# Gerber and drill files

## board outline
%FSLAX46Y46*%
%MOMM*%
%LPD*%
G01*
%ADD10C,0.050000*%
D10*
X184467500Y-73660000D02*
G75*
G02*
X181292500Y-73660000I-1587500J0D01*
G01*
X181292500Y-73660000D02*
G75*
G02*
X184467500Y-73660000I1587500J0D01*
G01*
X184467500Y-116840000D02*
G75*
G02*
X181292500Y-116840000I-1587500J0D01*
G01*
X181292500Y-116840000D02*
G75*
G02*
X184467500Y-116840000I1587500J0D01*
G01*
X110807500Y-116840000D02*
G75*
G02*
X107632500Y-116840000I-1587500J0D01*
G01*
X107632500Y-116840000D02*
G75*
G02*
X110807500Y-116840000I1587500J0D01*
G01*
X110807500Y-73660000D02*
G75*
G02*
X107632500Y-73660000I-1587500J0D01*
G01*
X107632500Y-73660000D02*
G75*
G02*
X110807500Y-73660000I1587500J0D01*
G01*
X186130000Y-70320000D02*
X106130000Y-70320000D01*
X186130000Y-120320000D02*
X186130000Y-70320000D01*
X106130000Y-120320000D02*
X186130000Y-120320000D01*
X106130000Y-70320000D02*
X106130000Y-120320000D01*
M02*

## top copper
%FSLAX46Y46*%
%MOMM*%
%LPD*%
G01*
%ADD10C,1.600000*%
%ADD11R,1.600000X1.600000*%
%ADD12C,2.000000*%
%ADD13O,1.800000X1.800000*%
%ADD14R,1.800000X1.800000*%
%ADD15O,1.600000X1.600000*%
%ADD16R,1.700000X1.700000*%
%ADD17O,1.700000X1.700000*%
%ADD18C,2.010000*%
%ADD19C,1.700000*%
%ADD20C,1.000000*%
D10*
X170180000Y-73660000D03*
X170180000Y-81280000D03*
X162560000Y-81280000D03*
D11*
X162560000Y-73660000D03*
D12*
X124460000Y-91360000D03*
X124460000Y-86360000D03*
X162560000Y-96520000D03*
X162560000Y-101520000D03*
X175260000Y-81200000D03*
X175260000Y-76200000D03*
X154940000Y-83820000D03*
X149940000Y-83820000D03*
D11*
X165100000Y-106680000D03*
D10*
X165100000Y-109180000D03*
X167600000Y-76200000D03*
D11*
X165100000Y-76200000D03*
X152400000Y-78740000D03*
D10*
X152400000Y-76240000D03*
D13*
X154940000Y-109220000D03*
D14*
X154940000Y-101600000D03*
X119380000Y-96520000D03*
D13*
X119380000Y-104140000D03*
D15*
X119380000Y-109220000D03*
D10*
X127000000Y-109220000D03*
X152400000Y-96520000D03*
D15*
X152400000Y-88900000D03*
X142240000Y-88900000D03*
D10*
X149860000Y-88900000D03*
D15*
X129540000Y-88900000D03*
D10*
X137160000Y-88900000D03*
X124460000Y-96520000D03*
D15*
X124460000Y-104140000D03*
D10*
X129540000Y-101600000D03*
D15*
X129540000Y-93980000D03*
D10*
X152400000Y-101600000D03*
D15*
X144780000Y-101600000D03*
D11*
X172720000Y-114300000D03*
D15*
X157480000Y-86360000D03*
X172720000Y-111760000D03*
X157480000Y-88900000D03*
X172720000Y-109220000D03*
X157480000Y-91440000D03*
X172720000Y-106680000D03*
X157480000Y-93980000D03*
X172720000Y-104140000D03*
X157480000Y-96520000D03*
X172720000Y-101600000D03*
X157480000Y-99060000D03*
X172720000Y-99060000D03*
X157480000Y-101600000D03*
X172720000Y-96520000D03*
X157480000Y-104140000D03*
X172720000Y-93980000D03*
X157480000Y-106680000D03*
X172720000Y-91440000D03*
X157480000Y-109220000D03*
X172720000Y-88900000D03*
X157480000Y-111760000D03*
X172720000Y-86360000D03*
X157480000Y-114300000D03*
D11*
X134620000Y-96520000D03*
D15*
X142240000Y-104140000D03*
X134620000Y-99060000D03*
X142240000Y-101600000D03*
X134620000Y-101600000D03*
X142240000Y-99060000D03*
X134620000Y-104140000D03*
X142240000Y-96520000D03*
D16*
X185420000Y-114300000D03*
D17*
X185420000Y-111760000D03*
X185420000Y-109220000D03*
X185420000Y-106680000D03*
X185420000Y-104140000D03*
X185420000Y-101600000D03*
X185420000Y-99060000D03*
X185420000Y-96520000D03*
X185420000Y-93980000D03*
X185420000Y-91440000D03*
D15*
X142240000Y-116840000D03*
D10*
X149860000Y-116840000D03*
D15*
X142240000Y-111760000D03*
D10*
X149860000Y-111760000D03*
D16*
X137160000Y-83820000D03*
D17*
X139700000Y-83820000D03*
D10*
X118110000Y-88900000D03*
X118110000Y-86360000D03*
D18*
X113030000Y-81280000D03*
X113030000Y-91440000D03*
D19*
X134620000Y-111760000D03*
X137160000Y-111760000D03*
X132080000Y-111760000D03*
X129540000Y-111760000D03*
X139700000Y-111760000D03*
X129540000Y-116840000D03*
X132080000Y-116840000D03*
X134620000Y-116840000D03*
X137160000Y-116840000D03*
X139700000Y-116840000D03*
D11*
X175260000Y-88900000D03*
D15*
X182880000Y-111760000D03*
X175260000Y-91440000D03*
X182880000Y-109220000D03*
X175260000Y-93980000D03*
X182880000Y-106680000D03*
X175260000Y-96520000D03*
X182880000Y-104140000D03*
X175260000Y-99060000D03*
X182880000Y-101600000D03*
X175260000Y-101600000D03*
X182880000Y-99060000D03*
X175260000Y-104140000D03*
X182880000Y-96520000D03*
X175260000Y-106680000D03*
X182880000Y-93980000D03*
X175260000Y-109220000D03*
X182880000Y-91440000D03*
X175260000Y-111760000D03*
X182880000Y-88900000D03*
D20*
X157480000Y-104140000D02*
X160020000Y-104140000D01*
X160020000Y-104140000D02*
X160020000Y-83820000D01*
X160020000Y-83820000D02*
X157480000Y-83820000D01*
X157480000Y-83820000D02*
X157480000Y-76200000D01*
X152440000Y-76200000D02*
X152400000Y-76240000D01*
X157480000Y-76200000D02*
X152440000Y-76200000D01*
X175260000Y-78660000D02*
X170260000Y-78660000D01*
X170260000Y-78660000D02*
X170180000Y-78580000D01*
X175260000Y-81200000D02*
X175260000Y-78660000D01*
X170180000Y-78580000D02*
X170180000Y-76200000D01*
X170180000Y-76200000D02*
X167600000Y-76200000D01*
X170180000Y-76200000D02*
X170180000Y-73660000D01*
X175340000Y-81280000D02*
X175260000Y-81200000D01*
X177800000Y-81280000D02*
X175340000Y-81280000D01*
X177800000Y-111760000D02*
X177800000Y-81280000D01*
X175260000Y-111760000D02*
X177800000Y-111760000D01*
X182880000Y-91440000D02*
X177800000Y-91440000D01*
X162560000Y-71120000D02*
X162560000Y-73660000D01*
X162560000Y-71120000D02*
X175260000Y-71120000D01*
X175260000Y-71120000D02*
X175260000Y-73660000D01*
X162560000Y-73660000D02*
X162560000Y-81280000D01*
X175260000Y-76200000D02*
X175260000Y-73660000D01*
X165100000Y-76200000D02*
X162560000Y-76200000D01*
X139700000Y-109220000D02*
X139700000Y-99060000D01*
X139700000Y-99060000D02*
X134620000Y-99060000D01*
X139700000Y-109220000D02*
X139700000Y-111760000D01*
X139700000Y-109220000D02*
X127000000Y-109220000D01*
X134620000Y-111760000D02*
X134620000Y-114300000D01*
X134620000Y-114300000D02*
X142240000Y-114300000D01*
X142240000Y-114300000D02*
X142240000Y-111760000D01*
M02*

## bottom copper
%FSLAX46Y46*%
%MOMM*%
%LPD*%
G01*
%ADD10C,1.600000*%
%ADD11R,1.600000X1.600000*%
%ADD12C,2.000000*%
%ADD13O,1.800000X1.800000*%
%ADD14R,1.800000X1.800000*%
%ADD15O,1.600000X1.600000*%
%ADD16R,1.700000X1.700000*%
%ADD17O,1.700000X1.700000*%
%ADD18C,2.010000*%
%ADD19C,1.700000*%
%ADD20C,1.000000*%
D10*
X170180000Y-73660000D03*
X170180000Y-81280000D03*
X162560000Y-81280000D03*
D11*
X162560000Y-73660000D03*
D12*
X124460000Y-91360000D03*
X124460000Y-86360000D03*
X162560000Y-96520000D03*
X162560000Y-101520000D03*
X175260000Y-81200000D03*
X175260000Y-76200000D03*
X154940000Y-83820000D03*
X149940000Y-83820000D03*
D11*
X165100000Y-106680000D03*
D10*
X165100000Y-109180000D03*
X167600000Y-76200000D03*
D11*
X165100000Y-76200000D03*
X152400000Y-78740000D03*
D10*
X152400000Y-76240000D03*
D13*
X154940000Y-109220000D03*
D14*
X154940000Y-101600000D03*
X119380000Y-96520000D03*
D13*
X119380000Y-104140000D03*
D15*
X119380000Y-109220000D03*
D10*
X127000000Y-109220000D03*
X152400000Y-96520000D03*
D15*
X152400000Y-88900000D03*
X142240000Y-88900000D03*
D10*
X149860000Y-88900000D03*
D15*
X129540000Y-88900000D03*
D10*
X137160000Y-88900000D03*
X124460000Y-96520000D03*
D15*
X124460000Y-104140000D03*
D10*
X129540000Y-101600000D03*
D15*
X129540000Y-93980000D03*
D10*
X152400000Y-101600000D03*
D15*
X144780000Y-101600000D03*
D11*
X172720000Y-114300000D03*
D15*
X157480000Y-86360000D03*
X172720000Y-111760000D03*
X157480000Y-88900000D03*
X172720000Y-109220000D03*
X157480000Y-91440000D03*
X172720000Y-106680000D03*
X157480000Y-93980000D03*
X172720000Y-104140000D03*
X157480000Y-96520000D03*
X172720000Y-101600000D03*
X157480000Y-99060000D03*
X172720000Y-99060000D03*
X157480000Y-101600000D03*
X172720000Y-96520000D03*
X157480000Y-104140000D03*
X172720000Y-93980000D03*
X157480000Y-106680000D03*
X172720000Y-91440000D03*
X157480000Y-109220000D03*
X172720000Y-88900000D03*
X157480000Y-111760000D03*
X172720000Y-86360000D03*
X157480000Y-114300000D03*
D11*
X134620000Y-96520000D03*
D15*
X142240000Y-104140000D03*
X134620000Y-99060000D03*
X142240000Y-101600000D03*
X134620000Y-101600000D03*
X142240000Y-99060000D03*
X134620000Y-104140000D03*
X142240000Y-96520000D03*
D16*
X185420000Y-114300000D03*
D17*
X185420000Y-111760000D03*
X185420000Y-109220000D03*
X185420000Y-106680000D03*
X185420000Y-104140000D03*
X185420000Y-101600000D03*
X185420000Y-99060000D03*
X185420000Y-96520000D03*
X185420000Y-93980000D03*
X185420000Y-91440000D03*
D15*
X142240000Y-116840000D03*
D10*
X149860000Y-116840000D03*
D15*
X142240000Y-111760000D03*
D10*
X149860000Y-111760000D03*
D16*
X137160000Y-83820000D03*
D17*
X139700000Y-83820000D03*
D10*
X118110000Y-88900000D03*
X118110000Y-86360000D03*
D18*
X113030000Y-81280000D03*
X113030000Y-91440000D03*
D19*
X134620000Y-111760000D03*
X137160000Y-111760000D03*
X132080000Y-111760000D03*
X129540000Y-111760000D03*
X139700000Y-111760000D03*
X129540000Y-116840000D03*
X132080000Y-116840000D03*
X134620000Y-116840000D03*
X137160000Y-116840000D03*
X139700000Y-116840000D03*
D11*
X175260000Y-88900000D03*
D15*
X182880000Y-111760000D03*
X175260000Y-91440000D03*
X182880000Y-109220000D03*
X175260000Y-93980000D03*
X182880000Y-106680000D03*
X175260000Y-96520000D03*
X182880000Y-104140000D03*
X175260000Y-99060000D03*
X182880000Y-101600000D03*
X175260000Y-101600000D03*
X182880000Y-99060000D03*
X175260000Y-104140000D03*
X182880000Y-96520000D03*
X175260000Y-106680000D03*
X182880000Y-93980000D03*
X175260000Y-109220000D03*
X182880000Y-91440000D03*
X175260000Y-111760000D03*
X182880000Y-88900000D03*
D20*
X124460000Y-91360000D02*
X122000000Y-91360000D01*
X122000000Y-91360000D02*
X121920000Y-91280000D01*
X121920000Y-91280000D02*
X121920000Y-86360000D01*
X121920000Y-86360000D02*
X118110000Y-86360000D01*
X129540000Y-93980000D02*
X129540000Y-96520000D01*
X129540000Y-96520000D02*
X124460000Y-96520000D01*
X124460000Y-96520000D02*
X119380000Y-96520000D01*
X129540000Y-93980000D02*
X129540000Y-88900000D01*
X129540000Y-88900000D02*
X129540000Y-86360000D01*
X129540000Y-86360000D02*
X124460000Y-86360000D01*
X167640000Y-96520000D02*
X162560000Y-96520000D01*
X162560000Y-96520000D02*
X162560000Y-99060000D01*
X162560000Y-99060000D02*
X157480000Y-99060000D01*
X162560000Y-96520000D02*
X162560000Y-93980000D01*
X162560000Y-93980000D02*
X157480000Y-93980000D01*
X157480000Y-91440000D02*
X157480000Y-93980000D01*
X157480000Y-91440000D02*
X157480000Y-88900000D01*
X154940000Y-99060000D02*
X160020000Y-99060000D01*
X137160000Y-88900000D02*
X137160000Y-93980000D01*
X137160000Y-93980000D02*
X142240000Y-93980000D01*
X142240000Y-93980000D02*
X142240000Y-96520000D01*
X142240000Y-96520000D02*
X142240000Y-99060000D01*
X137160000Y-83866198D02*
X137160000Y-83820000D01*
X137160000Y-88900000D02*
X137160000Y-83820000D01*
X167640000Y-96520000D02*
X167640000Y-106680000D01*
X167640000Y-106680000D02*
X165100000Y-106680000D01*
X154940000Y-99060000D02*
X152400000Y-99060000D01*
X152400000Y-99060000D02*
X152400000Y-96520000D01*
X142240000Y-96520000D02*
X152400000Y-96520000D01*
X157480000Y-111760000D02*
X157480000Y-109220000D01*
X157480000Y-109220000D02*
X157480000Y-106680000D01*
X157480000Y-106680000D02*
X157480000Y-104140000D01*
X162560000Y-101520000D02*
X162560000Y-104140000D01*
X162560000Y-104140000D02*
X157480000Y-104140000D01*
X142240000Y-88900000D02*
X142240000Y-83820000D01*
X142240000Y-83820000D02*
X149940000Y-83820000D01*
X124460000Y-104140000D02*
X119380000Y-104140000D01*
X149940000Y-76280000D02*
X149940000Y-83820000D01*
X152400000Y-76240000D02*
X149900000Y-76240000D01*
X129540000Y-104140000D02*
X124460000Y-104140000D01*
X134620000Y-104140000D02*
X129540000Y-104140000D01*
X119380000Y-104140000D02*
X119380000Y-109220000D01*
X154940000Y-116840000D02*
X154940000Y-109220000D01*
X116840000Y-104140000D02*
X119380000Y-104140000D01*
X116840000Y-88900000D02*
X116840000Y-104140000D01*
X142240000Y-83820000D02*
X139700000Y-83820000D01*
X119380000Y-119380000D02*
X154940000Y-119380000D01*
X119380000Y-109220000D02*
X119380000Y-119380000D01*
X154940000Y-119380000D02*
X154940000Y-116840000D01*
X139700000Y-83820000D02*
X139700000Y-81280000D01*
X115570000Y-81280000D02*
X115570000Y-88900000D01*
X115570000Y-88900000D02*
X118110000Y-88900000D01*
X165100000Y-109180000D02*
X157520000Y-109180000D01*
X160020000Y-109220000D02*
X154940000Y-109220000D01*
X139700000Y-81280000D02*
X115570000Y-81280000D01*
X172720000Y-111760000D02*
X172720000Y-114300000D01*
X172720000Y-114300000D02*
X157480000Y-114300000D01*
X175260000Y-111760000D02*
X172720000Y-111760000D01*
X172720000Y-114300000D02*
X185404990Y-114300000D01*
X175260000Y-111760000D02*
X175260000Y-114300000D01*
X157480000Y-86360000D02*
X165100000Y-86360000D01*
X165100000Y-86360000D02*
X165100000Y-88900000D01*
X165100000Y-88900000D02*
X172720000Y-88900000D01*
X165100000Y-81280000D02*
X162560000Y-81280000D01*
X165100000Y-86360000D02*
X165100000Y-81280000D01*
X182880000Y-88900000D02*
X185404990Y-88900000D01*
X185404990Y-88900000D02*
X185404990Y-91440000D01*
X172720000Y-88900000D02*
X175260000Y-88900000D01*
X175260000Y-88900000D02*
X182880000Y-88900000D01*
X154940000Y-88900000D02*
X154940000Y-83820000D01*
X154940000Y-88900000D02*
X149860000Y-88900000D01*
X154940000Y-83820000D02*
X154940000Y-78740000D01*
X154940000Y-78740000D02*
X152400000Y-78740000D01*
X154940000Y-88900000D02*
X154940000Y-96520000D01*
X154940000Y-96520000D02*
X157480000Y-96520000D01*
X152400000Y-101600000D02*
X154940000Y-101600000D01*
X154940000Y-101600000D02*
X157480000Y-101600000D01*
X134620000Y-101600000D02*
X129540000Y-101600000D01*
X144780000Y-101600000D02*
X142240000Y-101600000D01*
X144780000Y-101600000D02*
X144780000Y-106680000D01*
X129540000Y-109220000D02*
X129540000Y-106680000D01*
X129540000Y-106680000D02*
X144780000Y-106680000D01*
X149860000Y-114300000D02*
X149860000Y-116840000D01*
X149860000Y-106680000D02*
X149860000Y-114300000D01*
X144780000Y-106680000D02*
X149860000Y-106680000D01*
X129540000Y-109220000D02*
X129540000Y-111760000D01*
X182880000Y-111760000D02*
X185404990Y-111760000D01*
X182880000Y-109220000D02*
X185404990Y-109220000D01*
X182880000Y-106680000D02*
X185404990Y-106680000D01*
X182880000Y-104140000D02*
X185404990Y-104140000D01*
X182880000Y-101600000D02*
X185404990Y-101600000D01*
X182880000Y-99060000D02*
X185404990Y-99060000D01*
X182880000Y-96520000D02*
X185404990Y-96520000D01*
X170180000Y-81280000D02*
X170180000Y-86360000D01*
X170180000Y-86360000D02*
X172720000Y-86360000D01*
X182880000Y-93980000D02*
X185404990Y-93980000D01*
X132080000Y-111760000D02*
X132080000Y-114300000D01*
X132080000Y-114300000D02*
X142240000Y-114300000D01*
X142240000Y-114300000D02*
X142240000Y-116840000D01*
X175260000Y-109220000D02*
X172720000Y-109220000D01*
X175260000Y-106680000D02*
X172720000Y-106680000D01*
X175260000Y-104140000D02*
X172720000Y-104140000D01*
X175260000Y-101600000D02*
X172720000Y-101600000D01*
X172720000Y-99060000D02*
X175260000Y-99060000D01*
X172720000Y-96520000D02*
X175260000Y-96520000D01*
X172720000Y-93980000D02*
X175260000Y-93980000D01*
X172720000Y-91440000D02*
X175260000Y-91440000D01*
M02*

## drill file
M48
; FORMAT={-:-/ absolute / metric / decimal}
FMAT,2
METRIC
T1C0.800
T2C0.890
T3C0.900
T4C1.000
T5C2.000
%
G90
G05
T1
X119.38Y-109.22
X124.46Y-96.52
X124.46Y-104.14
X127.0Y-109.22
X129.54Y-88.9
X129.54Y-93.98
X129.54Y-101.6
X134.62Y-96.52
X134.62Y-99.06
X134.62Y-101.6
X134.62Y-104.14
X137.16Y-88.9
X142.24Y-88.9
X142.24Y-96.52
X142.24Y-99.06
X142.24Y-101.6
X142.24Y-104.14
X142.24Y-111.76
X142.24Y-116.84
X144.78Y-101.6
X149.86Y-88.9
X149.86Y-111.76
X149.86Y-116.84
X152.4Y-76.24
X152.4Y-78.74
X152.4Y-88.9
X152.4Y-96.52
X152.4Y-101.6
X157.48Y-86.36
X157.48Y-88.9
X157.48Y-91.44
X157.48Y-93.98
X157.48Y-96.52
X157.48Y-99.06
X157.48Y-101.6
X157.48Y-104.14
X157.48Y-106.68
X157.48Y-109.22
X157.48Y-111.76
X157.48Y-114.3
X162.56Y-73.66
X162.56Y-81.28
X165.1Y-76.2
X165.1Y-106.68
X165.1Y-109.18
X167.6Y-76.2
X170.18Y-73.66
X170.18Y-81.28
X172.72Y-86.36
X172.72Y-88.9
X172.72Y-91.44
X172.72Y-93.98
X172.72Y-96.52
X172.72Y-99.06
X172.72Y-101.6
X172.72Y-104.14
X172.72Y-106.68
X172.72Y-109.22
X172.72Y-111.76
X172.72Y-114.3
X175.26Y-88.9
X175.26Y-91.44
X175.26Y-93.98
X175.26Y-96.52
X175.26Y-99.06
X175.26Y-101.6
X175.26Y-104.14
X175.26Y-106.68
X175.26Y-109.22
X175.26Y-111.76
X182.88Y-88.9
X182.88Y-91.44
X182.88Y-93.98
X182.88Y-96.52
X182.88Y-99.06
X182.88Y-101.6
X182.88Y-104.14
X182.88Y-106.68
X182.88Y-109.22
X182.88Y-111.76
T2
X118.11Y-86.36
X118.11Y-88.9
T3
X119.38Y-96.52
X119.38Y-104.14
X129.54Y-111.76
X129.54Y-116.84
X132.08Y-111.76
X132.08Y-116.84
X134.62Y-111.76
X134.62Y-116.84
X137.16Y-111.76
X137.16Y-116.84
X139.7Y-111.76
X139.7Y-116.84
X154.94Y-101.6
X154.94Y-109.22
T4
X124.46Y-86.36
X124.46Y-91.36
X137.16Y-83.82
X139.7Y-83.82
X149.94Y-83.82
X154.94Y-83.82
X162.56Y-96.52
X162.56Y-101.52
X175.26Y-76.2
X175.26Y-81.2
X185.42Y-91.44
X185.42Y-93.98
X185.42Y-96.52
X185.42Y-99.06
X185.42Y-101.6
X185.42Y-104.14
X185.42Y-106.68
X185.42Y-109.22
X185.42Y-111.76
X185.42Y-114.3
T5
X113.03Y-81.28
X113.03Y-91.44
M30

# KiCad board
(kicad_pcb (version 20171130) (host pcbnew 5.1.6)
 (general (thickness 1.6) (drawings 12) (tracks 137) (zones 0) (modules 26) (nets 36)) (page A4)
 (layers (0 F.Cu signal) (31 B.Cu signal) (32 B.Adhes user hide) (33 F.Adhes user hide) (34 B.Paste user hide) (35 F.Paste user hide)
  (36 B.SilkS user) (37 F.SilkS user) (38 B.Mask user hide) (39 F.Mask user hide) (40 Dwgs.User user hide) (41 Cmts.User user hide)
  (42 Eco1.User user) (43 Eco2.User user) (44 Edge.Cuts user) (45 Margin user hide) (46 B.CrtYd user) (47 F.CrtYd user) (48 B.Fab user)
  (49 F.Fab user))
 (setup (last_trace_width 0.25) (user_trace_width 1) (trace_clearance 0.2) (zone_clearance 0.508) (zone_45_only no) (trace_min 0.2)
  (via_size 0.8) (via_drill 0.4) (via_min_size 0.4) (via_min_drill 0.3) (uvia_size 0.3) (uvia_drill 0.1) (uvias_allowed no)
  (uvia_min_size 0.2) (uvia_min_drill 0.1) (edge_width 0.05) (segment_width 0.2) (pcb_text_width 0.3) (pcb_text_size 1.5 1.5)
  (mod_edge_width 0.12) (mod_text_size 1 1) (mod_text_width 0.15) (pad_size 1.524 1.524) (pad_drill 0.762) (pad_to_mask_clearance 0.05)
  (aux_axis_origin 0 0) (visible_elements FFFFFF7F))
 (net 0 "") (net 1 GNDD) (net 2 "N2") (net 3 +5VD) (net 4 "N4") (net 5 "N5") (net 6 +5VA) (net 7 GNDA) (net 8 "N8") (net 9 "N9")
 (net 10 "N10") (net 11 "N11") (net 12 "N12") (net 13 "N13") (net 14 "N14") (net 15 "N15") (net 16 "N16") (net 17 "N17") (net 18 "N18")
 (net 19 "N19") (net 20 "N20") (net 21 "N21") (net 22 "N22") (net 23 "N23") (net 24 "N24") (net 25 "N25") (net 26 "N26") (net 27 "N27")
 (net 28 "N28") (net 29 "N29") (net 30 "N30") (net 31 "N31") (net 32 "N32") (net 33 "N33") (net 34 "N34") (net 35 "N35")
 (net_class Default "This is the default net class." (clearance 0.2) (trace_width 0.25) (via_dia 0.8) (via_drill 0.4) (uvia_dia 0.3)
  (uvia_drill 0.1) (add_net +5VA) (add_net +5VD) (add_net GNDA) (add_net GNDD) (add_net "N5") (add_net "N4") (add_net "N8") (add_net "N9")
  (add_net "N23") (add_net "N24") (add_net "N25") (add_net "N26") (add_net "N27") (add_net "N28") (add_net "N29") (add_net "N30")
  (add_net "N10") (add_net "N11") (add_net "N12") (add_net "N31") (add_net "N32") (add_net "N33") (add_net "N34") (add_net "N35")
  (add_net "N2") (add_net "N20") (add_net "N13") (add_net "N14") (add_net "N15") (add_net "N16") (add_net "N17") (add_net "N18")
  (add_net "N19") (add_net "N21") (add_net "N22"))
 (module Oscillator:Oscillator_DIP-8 (layer B.Cu) (at 162.56 73.66)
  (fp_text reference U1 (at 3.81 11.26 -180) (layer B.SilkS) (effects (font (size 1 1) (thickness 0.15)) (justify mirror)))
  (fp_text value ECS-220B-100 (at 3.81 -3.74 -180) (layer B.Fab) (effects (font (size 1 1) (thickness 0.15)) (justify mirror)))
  (pad 4 thru_hole circle (at 7.62 0) (size 1.6 1.6) (drill 0.8) (layers *.Cu *.Mask) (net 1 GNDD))
  (pad 5 thru_hole circle (at 7.62 7.62) (size 1.6 1.6) (drill 0.8) (layers *.Cu *.Mask) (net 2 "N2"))
  (pad 8 thru_hole circle (at 0 7.62) (size 1.6 1.6) (drill 0.8) (layers *.Cu *.Mask) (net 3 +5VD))
  (pad 1 thru_hole rect (at 0 0) (size 1.6 1.6) (drill 0.8) (layers *.Cu *.Mask) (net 3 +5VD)))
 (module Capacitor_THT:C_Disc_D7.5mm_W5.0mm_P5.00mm (layer F.Cu) (at 124.46 86.36 270)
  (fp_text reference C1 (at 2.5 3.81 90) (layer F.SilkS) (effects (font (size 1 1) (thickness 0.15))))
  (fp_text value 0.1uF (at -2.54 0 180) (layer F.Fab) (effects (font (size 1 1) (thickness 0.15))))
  (pad 2 thru_hole circle (at 5 0 270) (size 2 2) (drill 1) (layers *.Cu *.Mask) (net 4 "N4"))
  (pad 1 thru_hole circle (at 0 0 270) (size 2 2) (drill 1) (layers *.Cu *.Mask) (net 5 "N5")))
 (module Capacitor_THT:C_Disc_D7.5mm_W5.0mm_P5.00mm (layer B.Cu) (at 162.56 96.52 270)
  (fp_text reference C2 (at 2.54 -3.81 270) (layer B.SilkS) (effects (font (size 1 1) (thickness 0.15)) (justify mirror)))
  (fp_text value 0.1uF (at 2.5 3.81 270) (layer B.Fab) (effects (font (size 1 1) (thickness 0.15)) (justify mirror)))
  (pad 1 thru_hole circle (at 0 0 270) (size 2 2) (drill 1) (layers *.Cu *.Mask) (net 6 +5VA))
  (pad 2 thru_hole circle (at 5 0 270) (size 2 2) (drill 1) (layers *.Cu *.Mask) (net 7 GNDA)))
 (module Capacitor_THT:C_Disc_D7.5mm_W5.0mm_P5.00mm (layer F.Cu) (at 175.26 76.2 270)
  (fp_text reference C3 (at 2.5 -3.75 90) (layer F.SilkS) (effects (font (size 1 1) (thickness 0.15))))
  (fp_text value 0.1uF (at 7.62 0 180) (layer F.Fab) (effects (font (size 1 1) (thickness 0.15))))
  (pad 2 thru_hole circle (at 5 0 270) (size 2 2) (drill 1) (layers *.Cu *.Mask) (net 1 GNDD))
  (pad 1 thru_hole circle (at 0 0 270) (size 2 2) (drill 1) (layers *.Cu *.Mask) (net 3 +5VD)))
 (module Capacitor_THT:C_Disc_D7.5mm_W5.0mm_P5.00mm (layer F.Cu) (at 154.94 83.82 180)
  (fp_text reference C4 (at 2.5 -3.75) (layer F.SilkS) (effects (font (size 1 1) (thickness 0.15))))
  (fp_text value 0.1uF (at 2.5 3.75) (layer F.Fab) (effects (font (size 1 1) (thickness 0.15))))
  (pad 1 thru_hole circle (at 0 0 180) (size 2 2) (drill 1) (layers *.Cu *.Mask) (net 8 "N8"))
  (pad 2 thru_hole circle (at 5 0 180) (size 2 2) (drill 1) (layers *.Cu *.Mask) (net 7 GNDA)))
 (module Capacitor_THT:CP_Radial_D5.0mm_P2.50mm (layer B.Cu) (at 165.1 106.68 270)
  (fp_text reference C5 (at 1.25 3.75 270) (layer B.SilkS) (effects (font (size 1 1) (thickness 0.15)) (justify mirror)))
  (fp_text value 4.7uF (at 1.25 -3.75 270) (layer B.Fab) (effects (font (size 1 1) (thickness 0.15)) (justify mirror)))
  (pad 1 thru_hole rect (at 0 0 270) (size 1.6 1.6) (drill 0.8) (layers *.Cu *.Mask) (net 6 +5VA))
  (pad 2 thru_hole circle (at 2.5 0 270) (size 1.6 1.6) (drill 0.8) (layers *.Cu *.Mask) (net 7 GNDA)))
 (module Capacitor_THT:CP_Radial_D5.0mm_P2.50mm (layer F.Cu) (at 165.1 76.2)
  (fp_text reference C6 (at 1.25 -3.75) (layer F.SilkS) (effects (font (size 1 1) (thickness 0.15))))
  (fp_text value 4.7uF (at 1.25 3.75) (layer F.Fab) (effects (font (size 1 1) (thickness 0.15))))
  (pad 2 thru_hole circle (at 2.5 0) (size 1.6 1.6) (drill 0.8) (layers *.Cu *.Mask) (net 1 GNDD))
  (pad 1 thru_hole rect (at 0 0) (size 1.6 1.6) (drill 0.8) (layers *.Cu *.Mask) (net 3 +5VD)))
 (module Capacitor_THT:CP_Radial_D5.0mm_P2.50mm (layer F.Cu) (at 152.4 78.74 90)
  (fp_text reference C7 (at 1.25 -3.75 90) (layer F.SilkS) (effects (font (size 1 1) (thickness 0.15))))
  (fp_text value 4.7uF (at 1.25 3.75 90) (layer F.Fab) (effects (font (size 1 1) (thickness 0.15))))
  (pad 1 thru_hole rect (at 0 0 90) (size 1.6 1.6) (drill 0.8) (layers *.Cu *.Mask) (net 8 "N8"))
  (pad 2 thru_hole circle (at 2.5 0 90) (size 1.6 1.6) (drill 0.8) (layers *.Cu *.Mask) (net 7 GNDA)))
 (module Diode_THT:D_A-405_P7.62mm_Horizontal (layer F.Cu) (at 154.94 101.6 270)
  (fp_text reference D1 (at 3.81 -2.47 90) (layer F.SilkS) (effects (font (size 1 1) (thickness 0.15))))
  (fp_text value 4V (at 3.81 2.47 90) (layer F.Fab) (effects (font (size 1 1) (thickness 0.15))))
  (pad 2 thru_hole oval (at 7.62 0 270) (size 1.8 1.8) (drill 0.9) (layers *.Cu *.Mask) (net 7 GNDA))
  (pad 1 thru_hole rect (at 0 0 270) (size 1.8 1.8) (drill 0.9) (layers *.Cu *.Mask) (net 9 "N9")))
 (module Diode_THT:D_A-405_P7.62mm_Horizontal (layer F.Cu) (at 119.38 96.52 270)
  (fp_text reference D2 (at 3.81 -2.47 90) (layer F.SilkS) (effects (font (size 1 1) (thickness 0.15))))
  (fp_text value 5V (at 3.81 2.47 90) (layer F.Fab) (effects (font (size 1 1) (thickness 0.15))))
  (pad 1 thru_hole rect (at 0 0 270) (size 1.8 1.8) (drill 0.9) (layers *.Cu *.Mask) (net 5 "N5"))
  (pad 2 thru_hole oval (at 7.62 0 270) (size 1.8 1.8) (drill 0.9) (layers *.Cu *.Mask) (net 7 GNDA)))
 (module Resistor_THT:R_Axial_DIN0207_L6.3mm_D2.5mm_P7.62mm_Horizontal (layer F.Cu) (at 127 109.22 180)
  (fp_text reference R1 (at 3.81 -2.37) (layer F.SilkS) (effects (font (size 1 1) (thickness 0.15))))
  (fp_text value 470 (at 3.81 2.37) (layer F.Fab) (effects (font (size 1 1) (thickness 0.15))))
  (pad 2 thru_hole oval (at 7.62 0 180) (size 1.6 1.6) (drill 0.8) (layers *.Cu *.Mask) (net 7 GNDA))
  (pad 1 thru_hole circle (at 0 0 180) (size 1.6 1.6) (drill 0.8) (layers *.Cu *.Mask) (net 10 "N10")))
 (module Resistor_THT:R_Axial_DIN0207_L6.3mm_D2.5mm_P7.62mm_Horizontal (layer F.Cu) (at 152.4 96.52 90)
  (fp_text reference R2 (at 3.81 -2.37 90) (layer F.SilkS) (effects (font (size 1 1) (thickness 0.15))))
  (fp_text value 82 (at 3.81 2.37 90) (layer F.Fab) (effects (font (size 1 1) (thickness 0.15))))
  (pad 1 thru_hole circle (at 0 0 90) (size 1.6 1.6) (drill 0.8) (layers *.Cu *.Mask) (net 6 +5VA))
  (pad 2 thru_hole oval (at 7.62 0 90) (size 1.6 1.6) (drill 0.8) (layers *.Cu *.Mask) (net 8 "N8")))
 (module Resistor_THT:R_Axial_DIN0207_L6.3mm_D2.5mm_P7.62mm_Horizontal (layer F.Cu) (at 149.86 88.9 180)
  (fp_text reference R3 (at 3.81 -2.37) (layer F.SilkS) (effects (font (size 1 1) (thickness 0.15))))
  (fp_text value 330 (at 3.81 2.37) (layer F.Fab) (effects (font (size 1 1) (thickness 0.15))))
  (pad 2 thru_hole oval (at 7.62 0 180) (size 1.6 1.6) (drill 0.8) (layers *.Cu *.Mask) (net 7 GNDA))
  (pad 1 thru_hole circle (at 0 0 180) (size 1.6 1.6) (drill 0.8) (layers *.Cu *.Mask) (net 8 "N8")))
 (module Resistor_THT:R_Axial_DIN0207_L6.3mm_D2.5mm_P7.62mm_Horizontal (layer F.Cu) (at 137.16 88.9 180)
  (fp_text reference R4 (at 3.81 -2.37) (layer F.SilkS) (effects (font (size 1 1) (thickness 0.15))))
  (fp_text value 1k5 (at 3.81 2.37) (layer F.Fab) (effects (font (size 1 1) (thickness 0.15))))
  (pad 2 thru_hole oval (at 7.62 0 180) (size 1.6 1.6) (drill 0.8) (layers *.Cu *.Mask) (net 5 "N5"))
  (pad 1 thru_hole circle (at 0 0 180) (size 1.6 1.6) (drill 0.8) (layers *.Cu *.Mask) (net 6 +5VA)))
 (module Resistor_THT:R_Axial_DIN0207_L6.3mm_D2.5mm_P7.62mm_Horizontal (layer F.Cu) (at 124.46 96.52 270)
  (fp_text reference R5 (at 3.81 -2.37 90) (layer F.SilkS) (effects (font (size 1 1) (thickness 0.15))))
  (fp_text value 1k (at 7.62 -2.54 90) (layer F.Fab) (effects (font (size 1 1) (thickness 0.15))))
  (pad 1 thru_hole circle (at 0 0 270) (size 1.6 1.6) (drill 0.8) (layers *.Cu *.Mask) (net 5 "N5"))
  (pad 2 thru_hole oval (at 7.62 0 270) (size 1.6 1.6) (drill 0.8) (layers *.Cu *.Mask) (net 7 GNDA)))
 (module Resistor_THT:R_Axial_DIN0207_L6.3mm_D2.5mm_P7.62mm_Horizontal (layer F.Cu) (at 129.54 101.6 90)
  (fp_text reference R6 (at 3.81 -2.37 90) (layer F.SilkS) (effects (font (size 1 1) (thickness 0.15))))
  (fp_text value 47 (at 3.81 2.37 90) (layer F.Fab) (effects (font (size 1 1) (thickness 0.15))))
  (pad 1 thru_hole circle (at 0 0 90) (size 1.6 1.6) (drill 0.8) (layers *.Cu *.Mask) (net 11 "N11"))
  (pad 2 thru_hole oval (at 7.62 0 90) (size 1.6 1.6) (drill 0.8) (layers *.Cu *.Mask) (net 5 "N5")))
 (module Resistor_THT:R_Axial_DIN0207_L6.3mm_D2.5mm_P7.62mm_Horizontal (layer F.Cu) (at 152.4 101.6 180)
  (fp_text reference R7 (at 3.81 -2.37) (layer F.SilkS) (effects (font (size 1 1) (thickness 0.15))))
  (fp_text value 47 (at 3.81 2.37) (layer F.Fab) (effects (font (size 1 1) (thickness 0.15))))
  (pad 1 thru_hole circle (at 0 0 180) (size 1.6 1.6) (drill 0.8) (layers *.Cu *.Mask) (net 9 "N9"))
  (pad 2 thru_hole oval (at 7.62 0 180) (size 1.6 1.6) (drill 0.8) (layers *.Cu *.Mask) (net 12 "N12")))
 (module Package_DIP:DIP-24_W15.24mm (layer F.Cu) (at 172.72 114.3 180)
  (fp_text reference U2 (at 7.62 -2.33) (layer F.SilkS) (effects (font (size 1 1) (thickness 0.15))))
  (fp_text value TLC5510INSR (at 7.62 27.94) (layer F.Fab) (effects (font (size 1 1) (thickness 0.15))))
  (pad 1 thru_hole rect (at 0 0 180) (size 1.6 1.6) (drill 0.8) (layers *.Cu *.Mask) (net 1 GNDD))
  (pad 13 thru_hole oval (at 15.24 27.94 180) (size 1.6 1.6) (drill 0.8) (layers *.Cu *.Mask) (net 3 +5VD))
  (pad 2 thru_hole oval (at 0 2.54 180) (size 1.6 1.6) (drill 0.8) (layers *.Cu *.Mask) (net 1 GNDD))
  (pad 14 thru_hole oval (at 15.24 25.4 180) (size 1.6 1.6) (drill 0.8) (layers *.Cu *.Mask) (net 6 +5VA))
  (pad 3 thru_hole oval (at 0 5.08 180) (size 1.6 1.6) (drill 0.8) (layers *.Cu *.Mask) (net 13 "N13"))
  (pad 15 thru_hole oval (at 15.24 22.86 180) (size 1.6 1.6) (drill 0.8) (layers *.Cu *.Mask) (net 6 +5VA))
  (pad 4 thru_hole oval (at 0 7.62 180) (size 1.6 1.6) (drill 0.8) (layers *.Cu *.Mask) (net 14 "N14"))
  (pad 16 thru_hole oval (at 15.24 20.32 180) (size 1.6 1.6) (drill 0.8) (layers *.Cu *.Mask) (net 6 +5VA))
  (pad 5 thru_hole oval (at 0 10.16 180) (size 1.6 1.6) (drill 0.8) (layers *.Cu *.Mask) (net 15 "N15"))
  (pad 17 thru_hole oval (at 15.24 17.78 180) (size 1.6 1.6) (drill 0.8) (layers *.Cu *.Mask) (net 8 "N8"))
  (pad 6 thru_hole oval (at 0 12.7 180) (size 1.6 1.6) (drill 0.8) (layers *.Cu *.Mask) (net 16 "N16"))
  (pad 18 thru_hole oval (at 15.24 15.24 180) (size 1.6 1.6) (drill 0.8) (layers *.Cu *.Mask) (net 6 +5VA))
  (pad 7 thru_hole oval (at 0 15.24 180) (size 1.6 1.6) (drill 0.8) (layers *.Cu *.Mask) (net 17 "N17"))
  (pad 19 thru_hole oval (at 15.24 12.7 180) (size 1.6 1.6) (drill 0.8) (layers *.Cu *.Mask) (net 9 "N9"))
  (pad 8 thru_hole oval (at 0 17.78 180) (size 1.6 1.6) (drill 0.8) (layers *.Cu *.Mask) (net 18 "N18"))
  (pad 20 thru_hole oval (at 15.24 10.16 180) (size 1.6 1.6) (drill 0.8) (layers *.Cu *.Mask) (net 7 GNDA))
  (pad 9 thru_hole oval (at 0 20.32 180) (size 1.6 1.6) (drill 0.8) (layers *.Cu *.Mask) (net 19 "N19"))
  (pad 21 thru_hole oval (at 15.24 7.62 180) (size 1.6 1.6) (drill 0.8) (layers *.Cu *.Mask) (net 7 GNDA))
  (pad 10 thru_hole oval (at 0 22.86 180) (size 1.6 1.6) (drill 0.8) (layers *.Cu *.Mask) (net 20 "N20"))
  (pad 22 thru_hole oval (at 15.24 5.08 180) (size 1.6 1.6) (drill 0.8) (layers *.Cu *.Mask) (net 7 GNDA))
  (pad 11 thru_hole oval (at 0 25.4 180) (size 1.6 1.6) (drill 0.8) (layers *.Cu *.Mask) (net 3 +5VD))
  (pad 23 thru_hole oval (at 15.24 2.54 180) (size 1.6 1.6) (drill 0.8) (layers *.Cu *.Mask) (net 7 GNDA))
  (pad 12 thru_hole oval (at 0 27.94 180) (size 1.6 1.6) (drill 0.8) (layers *.Cu *.Mask) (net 2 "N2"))
  (pad 24 thru_hole oval (at 15.24 0 180) (size 1.6 1.6) (drill 0.8) (layers *.Cu *.Mask) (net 1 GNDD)))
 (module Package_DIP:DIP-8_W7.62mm (layer F.Cu) (at 134.62 96.52)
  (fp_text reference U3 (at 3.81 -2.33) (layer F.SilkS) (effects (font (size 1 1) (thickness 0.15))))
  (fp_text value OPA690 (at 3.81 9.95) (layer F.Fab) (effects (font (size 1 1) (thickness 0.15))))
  (pad 1 thru_hole rect (at 0 0) (size 1.6 1.6) (drill 0.8) (layers *.Cu *.Mask) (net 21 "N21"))
  (pad 5 thru_hole oval (at 7.62 7.62) (size 1.6 1.6) (drill 0.8) (layers *.Cu *.Mask) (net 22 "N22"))
  (pad 2 thru_hole oval (at 0 2.54) (size 1.6 1.6) (drill 0.8) (layers *.Cu *.Mask) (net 10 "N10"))
  (pad 6 thru_hole oval (at 7.62 5.08) (size 1.6 1.6) (drill 0.8) (layers *.Cu *.Mask) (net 12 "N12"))
  (pad 3 thru_hole oval (at 0 5.08) (size 1.6 1.6) (drill 0.8) (layers *.Cu *.Mask) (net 11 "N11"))
  (pad 7 thru_hole oval (at 7.62 2.54) (size 1.6 1.6) (drill 0.8) (layers *.Cu *.Mask) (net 6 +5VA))
  (pad 4 thru_hole oval (at 0 7.62) (size 1.6 1.6) (drill 0.8) (layers *.Cu *.Mask) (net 7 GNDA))
  (pad 8 thru_hole oval (at 7.62 0) (size 1.6 1.6) (drill 0.8) (layers *.Cu *.Mask) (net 6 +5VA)))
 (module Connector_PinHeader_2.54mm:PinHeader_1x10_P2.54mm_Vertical (layer F.Cu) (at 185.42 114.3 180)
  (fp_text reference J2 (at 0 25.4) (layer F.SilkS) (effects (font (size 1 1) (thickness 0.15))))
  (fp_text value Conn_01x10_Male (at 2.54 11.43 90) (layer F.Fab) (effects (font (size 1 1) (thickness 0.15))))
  (pad 1 thru_hole rect (at 0 0 180) (size 1.7 1.7) (drill 1) (layers *.Cu *.Mask) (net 1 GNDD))
  (pad 2 thru_hole oval (at 0 2.54 180) (size 1.7 1.7) (drill 1) (layers *.Cu *.Mask) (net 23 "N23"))
  (pad 3 thru_hole oval (at 0 5.08 180) (size 1.7 1.7) (drill 1) (layers *.Cu *.Mask) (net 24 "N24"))
  (pad 4 thru_hole oval (at 0 7.62 180) (size 1.7 1.7) (drill 1) (layers *.Cu *.Mask) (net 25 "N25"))
  (pad 5 thru_hole oval (at 0 10.16 180) (size 1.7 1.7) (drill 1) (layers *.Cu *.Mask) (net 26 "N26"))
  (pad 6 thru_hole oval (at 0 12.7 180) (size 1.7 1.7) (drill 1) (layers *.Cu *.Mask) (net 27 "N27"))
  (pad 7 thru_hole oval (at 0 15.24 180) (size 1.7 1.7) (drill 1) (layers *.Cu *.Mask) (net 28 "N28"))
  (pad 8 thru_hole oval (at 0 17.78 180) (size 1.7 1.7) (drill 1) (layers *.Cu *.Mask) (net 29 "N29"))
  (pad 9 thru_hole oval (at 0 20.32 180) (size 1.7 1.7) (drill 1) (layers *.Cu *.Mask) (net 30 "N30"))
  (pad 10 thru_hole oval (at 0 22.86 180) (size 1.7 1.7) (drill 1) (layers *.Cu *.Mask) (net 3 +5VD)))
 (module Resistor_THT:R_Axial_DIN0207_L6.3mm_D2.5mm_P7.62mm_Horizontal (layer F.Cu) (at 149.86 116.84 180)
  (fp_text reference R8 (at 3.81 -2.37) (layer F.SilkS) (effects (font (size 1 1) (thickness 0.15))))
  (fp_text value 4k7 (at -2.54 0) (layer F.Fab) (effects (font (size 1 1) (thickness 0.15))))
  (pad 2 thru_hole oval (at 7.62 0 180) (size 1.6 1.6) (drill 0.8) (layers *.Cu *.Mask) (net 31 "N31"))
  (pad 1 thru_hole circle (at 0 0 180) (size 1.6 1.6) (drill 0.8) (layers *.Cu *.Mask) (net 12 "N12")))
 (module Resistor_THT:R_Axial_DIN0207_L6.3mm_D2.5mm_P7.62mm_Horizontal (layer F.Cu) (at 149.86 111.76 180)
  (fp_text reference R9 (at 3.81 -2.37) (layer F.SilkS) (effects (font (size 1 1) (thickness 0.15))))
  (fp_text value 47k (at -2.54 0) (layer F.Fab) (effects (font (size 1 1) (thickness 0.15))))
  (pad 2 thru_hole oval (at 7.62 0 180) (size 1.6 1.6) (drill 0.8) (layers *.Cu *.Mask) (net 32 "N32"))
  (pad 1 thru_hole circle (at 0 0 180) (size 1.6 1.6) (drill 0.8) (layers *.Cu *.Mask) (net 12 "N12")))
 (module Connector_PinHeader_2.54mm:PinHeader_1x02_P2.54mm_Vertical (layer F.Cu) (at 137.16 83.82 90)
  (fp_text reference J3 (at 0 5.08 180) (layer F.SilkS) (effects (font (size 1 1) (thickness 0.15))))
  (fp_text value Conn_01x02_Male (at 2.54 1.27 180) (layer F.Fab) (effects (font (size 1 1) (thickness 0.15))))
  (pad 1 thru_hole rect (at 0 0 90) (size 1.7 1.7) (drill 1) (layers *.Cu *.Mask) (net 6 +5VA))
  (pad 2 thru_hole oval (at 0 2.54 90) (size 1.7 1.7) (drill 1) (layers *.Cu *.Mask) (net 7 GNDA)))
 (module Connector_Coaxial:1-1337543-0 (layer F.Cu) (at 118.11 86.36 90)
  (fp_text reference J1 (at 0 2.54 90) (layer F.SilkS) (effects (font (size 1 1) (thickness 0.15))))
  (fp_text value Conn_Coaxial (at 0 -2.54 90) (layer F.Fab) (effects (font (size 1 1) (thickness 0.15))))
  (pad 2 thru_hole circle (at -2.54 0 90) (size 1.6 1.6) (drill 0.89) (layers *.Cu *.Mask) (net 7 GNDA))
  (pad 1 thru_hole circle (at 0 0 90) (size 1.6 1.6) (drill 0.89) (layers *.Cu *.Mask) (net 4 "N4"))
  (pad 4 thru_hole circle (at 5.08 -5.08 90) (size 2.01 2.01) (drill 2) (layers *.Cu *.Mask))
  (pad 3 thru_hole circle (at -5.08 -5.08 90) (size 2.01 2.01) (drill 2) (layers *.Cu *.Mask)))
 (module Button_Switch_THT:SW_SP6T (layer F.Cu) (at 134.62 111.76)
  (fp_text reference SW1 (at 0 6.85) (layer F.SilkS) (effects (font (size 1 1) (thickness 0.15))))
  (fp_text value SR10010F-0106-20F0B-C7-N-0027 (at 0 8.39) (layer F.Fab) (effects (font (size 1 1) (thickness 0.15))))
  (pad 3 thru_hole circle (at 0 0) (size 1.7 1.7) (drill 0.9) (layers *.Cu *.Mask) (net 32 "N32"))
  (pad 4 thru_hole circle (at 2.54 0) (size 1.7 1.7) (drill 0.9) (layers *.Cu *.Mask) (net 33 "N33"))
  (pad 2 thru_hole circle (at -2.54 0) (size 1.7 1.7) (drill 0.9) (layers *.Cu *.Mask) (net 31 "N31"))
  (pad 1 thru_hole circle (at -5.08 0) (size 1.7 1.7) (drill 0.9) (layers *.Cu *.Mask) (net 12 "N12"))
  (pad 5 thru_hole circle (at 5.08 0) (size 1.7 1.7) (drill 0.9) (layers *.Cu *.Mask) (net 10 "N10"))
  (pad 6 thru_hole circle (at -5.08 5.08) (size 1.7 1.7) (drill 0.9) (layers *.Cu *.Mask) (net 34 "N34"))
  (pad 7 thru_hole circle (at -2.54 5.08) (size 1.7 1.7) (drill 0.9) (layers *.Cu *.Mask) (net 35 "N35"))
  (pad 8 thru_hole circle (at 0 5.08) (size 1.7 1.7) (drill 0.9) (layers *.Cu *.Mask))
  (pad 9 thru_hole circle (at 2.54 5.08) (size 1.7 1.7) (drill 0.9) (layers *.Cu *.Mask))
  (pad 10 thru_hole circle (at 5.08 5.08) (size 1.7 1.7) (drill 0.9) (layers *.Cu *.Mask)))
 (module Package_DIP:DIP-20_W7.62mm (layer F.Cu) (at 175.26 88.9)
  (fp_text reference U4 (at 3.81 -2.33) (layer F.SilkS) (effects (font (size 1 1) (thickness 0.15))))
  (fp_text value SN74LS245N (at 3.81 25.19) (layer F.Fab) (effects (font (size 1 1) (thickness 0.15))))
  (pad 1 thru_hole rect (at 0 0) (size 1.6 1.6) (drill 0.8) (layers *.Cu *.Mask) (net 3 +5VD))
  (pad 11 thru_hole oval (at 7.62 22.86) (size 1.6 1.6) (drill 0.8) (layers *.Cu *.Mask) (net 23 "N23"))
  (pad 2 thru_hole oval (at 0 2.54) (size 1.6 1.6) (drill 0.8) (layers *.Cu *.Mask) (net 20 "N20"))
  (pad 12 thru_hole oval (at 7.62 20.32) (size 1.6 1.6) (drill 0.8) (layers *.Cu *.Mask) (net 24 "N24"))
  (pad 3 thru_hole oval (at 0 5.08) (size 1.6 1.6) (drill 0.8) (layers *.Cu *.Mask) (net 19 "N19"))
  (pad 13 thru_hole oval (at 7.62 17.78) (size 1.6 1.6) (drill 0.8) (layers *.Cu *.Mask) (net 25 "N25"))
  (pad 4 thru_hole oval (at 0 7.62) (size 1.6 1.6) (drill 0.8) (layers *.Cu *.Mask) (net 18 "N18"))
  (pad 14 thru_hole oval (at 7.62 15.24) (size 1.6 1.6) (drill 0.8) (layers *.Cu *.Mask) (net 26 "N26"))
  (pad 5 thru_hole oval (at 0 10.16) (size 1.6 1.6) (drill 0.8) (layers *.Cu *.Mask) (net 17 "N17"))
  (pad 15 thru_hole oval (at 7.62 12.7) (size 1.6 1.6) (drill 0.8) (layers *.Cu *.Mask) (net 27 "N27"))
  (pad 6 thru_hole oval (at 0 12.7) (size 1.6 1.6) (drill 0.8) (layers *.Cu *.Mask) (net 16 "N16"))
  (pad 16 thru_hole oval (at 7.62 10.16) (size 1.6 1.6) (drill 0.8) (layers *.Cu *.Mask) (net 28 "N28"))
  (pad 7 thru_hole oval (at 0 15.24) (size 1.6 1.6) (drill 0.8) (layers *.Cu *.Mask) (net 15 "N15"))
  (pad 17 thru_hole oval (at 7.62 7.62) (size 1.6 1.6) (drill 0.8) (layers *.Cu *.Mask) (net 29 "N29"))
  (pad 8 thru_hole oval (at 0 17.78) (size 1.6 1.6) (drill 0.8) (layers *.Cu *.Mask) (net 14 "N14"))
  (pad 18 thru_hole oval (at 7.62 5.08) (size 1.6 1.6) (drill 0.8) (layers *.Cu *.Mask) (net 30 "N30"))
  (pad 9 thru_hole oval (at 0 20.32) (size 1.6 1.6) (drill 0.8) (layers *.Cu *.Mask) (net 13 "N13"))
  (pad 19 thru_hole oval (at 7.62 2.54) (size 1.6 1.6) (drill 0.8) (layers *.Cu *.Mask) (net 1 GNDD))
  (pad 10 thru_hole oval (at 0 22.86) (size 1.6 1.6) (drill 0.8) (layers *.Cu *.Mask) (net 1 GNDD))
  (pad 20 thru_hole oval (at 7.62 0) (size 1.6 1.6) (drill 0.8) (layers *.Cu *.Mask) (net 3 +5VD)))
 (gr_circle (center 182.88 73.66) (end 184.4675 73.66) (layer Edge.Cuts) (width 0.05))
 (gr_circle (center 182.88 116.84) (end 184.4675 116.84) (layer Edge.Cuts) (width 0.05))
 (gr_circle (center 109.22 116.84) (end 110.8075 116.84) (layer Edge.Cuts) (width 0.05))
 (gr_circle (center 109.22 73.66) (end 110.8075 73.66) (layer Edge.Cuts) (width 0.05))
 (gr_line (start 186.13 70.32) (end 106.13 70.32) (layer Edge.Cuts) (width 0.05))
 (gr_line (start 186.13 120.32) (end 186.13 70.32) (layer Edge.Cuts) (width 0.05))
 (gr_line (start 106.13 120.32) (end 186.13 120.32) (layer Edge.Cuts) (width 0.05))
 (gr_line (start 106.13 70.32) (end 106.13 120.32) (layer Edge.Cuts) (width 0.05))
 (segment (start 124.46 91.36) (end 122 91.36) (width 1) (layer B.Cu) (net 4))
 (segment (start 122 91.36) (end 121.92 91.28) (width 1) (layer B.Cu) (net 4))
 (segment (start 121.92 91.28) (end 121.92 86.36) (width 1) (layer B.Cu) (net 4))
 (segment (start 121.92 86.36) (end 118.11 86.36) (width 1) (layer B.Cu) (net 4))
 (segment (start 129.54 93.98) (end 129.54 96.52) (width 1) (layer B.Cu) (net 5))
 (segment (start 129.54 96.52) (end 124.46 96.52) (width 1) (layer B.Cu) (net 5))
 (segment (start 124.46 96.52) (end 119.38 96.52) (width 1) (layer B.Cu) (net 5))
 (segment (start 129.54 93.98) (end 129.54 88.9) (width 1) (layer B.Cu) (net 5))
 (segment (start 129.54 88.9) (end 129.54 86.36) (width 1) (layer B.Cu) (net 5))
 (segment (start 129.54 86.36) (end 124.46 86.36) (width 1) (layer B.Cu) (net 5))
 (segment (start 167.64 96.52) (end 162.56 96.52) (width 1) (layer B.Cu) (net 6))
 (segment (start 162.56 96.52) (end 162.56 99.06) (width 1) (layer B.Cu) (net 6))
 (segment (start 162.56 99.06) (end 157.48 99.06) (width 1) (layer B.Cu) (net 6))
 (segment (start 162.56 96.52) (end 162.56 93.98) (width 1) (layer B.Cu) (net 6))
 (segment (start 162.56 93.98) (end 157.48 93.98) (width 1) (layer B.Cu) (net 6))
 (segment (start 157.48 91.44) (end 157.48 93.98) (width 1) (layer B.Cu) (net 6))
 (segment (start 157.48 91.44) (end 157.48 88.9) (width 1) (layer B.Cu) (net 6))
 (segment (start 154.94 99.06) (end 160.02 99.06) (width 1) (layer B.Cu) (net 6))
 (segment (start 137.16 88.9) (end 137.16 93.98) (width 1) (layer B.Cu) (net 6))
 (segment (start 137.16 93.98) (end 142.24 93.98) (width 1) (layer B.Cu) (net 6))
 (segment (start 142.24 93.98) (end 142.24 96.52) (width 1) (layer B.Cu) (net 6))
 (segment (start 142.24 96.52) (end 142.24 99.06) (width 1) (layer B.Cu) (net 6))
 (segment (start 137.16 83.866198) (end 137.16 83.82) (width 1) (layer B.Cu) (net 6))
 (segment (start 137.16 88.9) (end 137.16 83.82) (width 1) (layer B.Cu) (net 6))
 (segment (start 167.64 96.52) (end 167.64 106.68) (width 1) (layer B.Cu) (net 6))
 (segment (start 167.64 106.68) (end 165.1 106.68) (width 1) (layer B.Cu) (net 6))
 (segment (start 154.94 99.06) (end 152.4 99.06) (width 1) (layer B.Cu) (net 6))
 (segment (start 152.4 99.06) (end 152.4 96.52) (width 1) (layer B.Cu) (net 6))
 (segment (start 142.24 96.52) (end 152.4 96.52) (width 1) (layer B.Cu) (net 6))
 (segment (start 157.48 111.76) (end 157.48 109.22) (width 1) (layer B.Cu) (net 7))
 (segment (start 157.48 109.22) (end 157.48 106.68) (width 1) (layer B.Cu) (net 7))
 (segment (start 157.48 106.68) (end 157.48 104.14) (width 1) (layer B.Cu) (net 7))
 (segment (start 162.56 101.52) (end 162.56 104.14) (width 1) (layer B.Cu) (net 7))
 (segment (start 162.56 104.14) (end 157.48 104.14) (width 1) (layer B.Cu) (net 7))
 (segment (start 142.24 88.9) (end 142.24 83.82) (width 1) (layer B.Cu) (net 7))
 (segment (start 142.24 83.82) (end 149.94 83.82) (width 1) (layer B.Cu) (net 7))
 (segment (start 124.46 104.14) (end 119.38 104.14) (width 1) (layer B.Cu) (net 7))
 (segment (start 149.94 76.28) (end 149.94 83.82) (width 1) (layer B.Cu) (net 7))
 (segment (start 152.4 76.24) (end 149.9 76.24) (width 1) (layer B.Cu) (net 7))
 (segment (start 129.54 104.14) (end 124.46 104.14) (width 1) (layer B.Cu) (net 7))
 (segment (start 134.62 104.14) (end 129.54 104.14) (width 1) (layer B.Cu) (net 7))
 (segment (start 119.38 104.14) (end 119.38 109.22) (width 1) (layer B.Cu) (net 7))
 (segment (start 154.94 116.84) (end 154.94 109.22) (width 1) (layer B.Cu) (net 7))
 (segment (start 116.84 104.14) (end 119.38 104.14) (width 1) (layer B.Cu) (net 7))
 (segment (start 116.84 88.9) (end 116.84 104.14) (width 1) (layer B.Cu) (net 7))
 (segment (start 142.24 83.82) (end 139.7 83.82) (width 1) (layer B.Cu) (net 7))
 (segment (start 119.38 119.38) (end 154.94 119.38) (width 1) (layer B.Cu) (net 7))
 (segment (start 119.38 109.22) (end 119.38 119.38) (width 1) (layer B.Cu) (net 7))
 (segment (start 154.94 119.38) (end 154.94 116.84) (width 1) (layer B.Cu) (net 7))
 (segment (start 139.7 83.82) (end 139.7 81.28) (width 1) (layer B.Cu) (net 7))
 (segment (start 115.57 81.28) (end 115.57 88.9) (width 1) (layer B.Cu) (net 7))
 (segment (start 115.57 88.9) (end 118.11 88.9) (width 1) (layer B.Cu) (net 7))
 (segment (start 165.1 109.18) (end 157.52 109.18) (width 1) (layer B.Cu) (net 7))
 (segment (start 160.02 109.22) (end 154.94 109.22) (width 1) (layer B.Cu) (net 7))
 (segment (start 157.48 104.14) (end 160.02 104.14) (width 1) (layer F.Cu) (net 7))
 (segment (start 160.02 104.14) (end 160.02 83.82) (width 1) (layer F.Cu) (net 7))
 (segment (start 160.02 83.82) (end 157.48 83.82) (width 1) (layer F.Cu) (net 7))
 (segment (start 157.48 83.82) (end 157.48 76.2) (width 1) (layer F.Cu) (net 7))
 (segment (start 152.44 76.2) (end 152.4 76.24) (width 1) (layer F.Cu) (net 7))
 (segment (start 157.48 76.2) (end 152.44 76.2) (width 1) (layer F.Cu) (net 7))
 (segment (start 139.7 81.28) (end 115.57 81.28) (width 1) (layer B.Cu) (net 7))
 (segment (start 172.72 111.76) (end 172.72 114.3) (width 1) (layer B.Cu) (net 1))
 (segment (start 172.72 114.3) (end 157.48 114.3) (width 1) (layer B.Cu) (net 1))
 (segment (start 175.26 78.66) (end 170.26 78.66) (width 1) (layer F.Cu) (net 1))
 (segment (start 170.26 78.66) (end 170.18 78.58) (width 1) (layer F.Cu) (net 1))
 (segment (start 175.26 81.2) (end 175.26 78.66) (width 1) (layer F.Cu) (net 1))
 (segment (start 170.18 78.58) (end 170.18 76.2) (width 1) (layer F.Cu) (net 1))
 (segment (start 170.18 76.2) (end 167.6 76.2) (width 1) (layer F.Cu) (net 1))
 (segment (start 170.18 76.2) (end 170.18 73.66) (width 1) (layer F.Cu) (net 1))
 (segment (start 175.34 81.28) (end 175.26 81.2) (width 1) (layer F.Cu) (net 1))
 (segment (start 177.8 81.28) (end 175.34 81.28) (width 1) (layer F.Cu) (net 1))
 (segment (start 177.8 111.76) (end 177.8 81.28) (width 1) (layer F.Cu) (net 1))
 (segment (start 175.26 111.76) (end 177.8 111.76) (width 1) (layer F.Cu) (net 1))
 (segment (start 182.88 91.44) (end 177.8 91.44) (width 1) (layer F.Cu) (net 1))
 (segment (start 175.26 111.76) (end 172.72 111.76) (width 1) (layer B.Cu) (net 1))
 (segment (start 172.72 114.3) (end 185.40499 114.3) (width 1) (layer B.Cu) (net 1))
 (segment (start 175.26 111.76) (end 175.26 114.3) (width 1) (layer B.Cu) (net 1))
 (segment (start 157.48 86.36) (end 165.1 86.36) (width 1) (layer B.Cu) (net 3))
 (segment (start 165.1 86.36) (end 165.1 88.9) (width 1) (layer B.Cu) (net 3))
 (segment (start 165.1 88.9) (end 172.72 88.9) (width 1) (layer B.Cu) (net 3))
 (segment (start 162.56 71.12) (end 162.56 73.66) (width 1) (layer F.Cu) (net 3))
 (segment (start 162.56 71.12) (end 175.26 71.12) (width 1) (layer F.Cu) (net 3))
 (segment (start 175.26 71.12) (end 175.26 73.66) (width 1) (layer F.Cu) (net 3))
 (segment (start 162.56 73.66) (end 162.56 81.28) (width 1) (layer F.Cu) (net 3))
 (segment (start 175.26 76.2) (end 175.26 73.66) (width 1) (layer F.Cu) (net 3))
 (segment (start 165.1 81.28) (end 162.56 81.28) (width 1) (layer B.Cu) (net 3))
 (segment (start 165.1 86.36) (end 165.1 81.28) (width 1) (layer B.Cu) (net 3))
 (segment (start 165.1 76.2) (end 162.56 76.2) (width 1) (layer F.Cu) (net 3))
 (segment (start 182.88 88.9) (end 185.40499 88.9) (width 1) (layer B.Cu) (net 3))
 (segment (start 185.40499 88.9) (end 185.40499 91.44) (width 1) (layer B.Cu) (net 3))
 (segment (start 172.72 88.9) (end 175.26 88.9) (width 1) (layer B.Cu) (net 3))
 (segment (start 175.26 88.9) (end 182.88 88.9) (width 1) (layer B.Cu) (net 3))
 (segment (start 154.94 88.9) (end 154.94 83.82) (width 1) (layer B.Cu) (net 8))
 (segment (start 154.94 88.9) (end 149.86 88.9) (width 1) (layer B.Cu) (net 8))
 (segment (start 154.94 83.82) (end 154.94 78.74) (width 1) (layer B.Cu) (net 8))
 (segment (start 154.94 78.74) (end 152.4 78.74) (width 1) (layer B.Cu) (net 8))
 (segment (start 154.94 88.9) (end 154.94 96.52) (width 1) (layer B.Cu) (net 8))
 (segment (start 154.94 96.52) (end 157.48 96.52) (width 1) (layer B.Cu) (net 8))
 (segment (start 152.4 101.6) (end 154.94 101.6) (width 1) (layer B.Cu) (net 9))
 (segment (start 154.94 101.6) (end 157.48 101.6) (width 1) (layer B.Cu) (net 9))
 (segment (start 139.7 109.22) (end 139.7 99.06) (width 1) (layer F.Cu) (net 10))
 (segment (start 139.7 99.06) (end 134.62 99.06) (width 1) (layer F.Cu) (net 10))
 (segment (start 139.7 109.22) (end 139.7 111.76) (width 1) (layer F.Cu) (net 10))
 (segment (start 139.7 109.22) (end 127 109.22) (width 1) (layer F.Cu) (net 10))
 (segment (start 134.62 101.6) (end 129.54 101.6) (width 1) (layer B.Cu) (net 11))
 (segment (start 144.78 101.6) (end 142.24 101.6) (width 1) (layer B.Cu) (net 12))
 (segment (start 144.78 101.6) (end 144.78 106.68) (width 1) (layer B.Cu) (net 12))
 (segment (start 129.54 109.22) (end 129.54 106.68) (width 1) (layer B.Cu) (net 12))
 (segment (start 129.54 106.68) (end 144.78 106.68) (width 1) (layer B.Cu) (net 12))
 (segment (start 149.86 114.3) (end 149.86 116.84) (width 1) (layer B.Cu) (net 12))
 (segment (start 149.86 106.68) (end 149.86 114.3) (width 1) (layer B.Cu) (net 12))
 (segment (start 144.78 106.68) (end 149.86 106.68) (width 1) (layer B.Cu) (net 12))
 (segment (start 129.54 109.22) (end 129.54 111.76) (width 1) (layer B.Cu) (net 12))
 (segment (start 182.88 111.76) (end 185.40499 111.76) (width 1) (layer B.Cu) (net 23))
 (segment (start 182.88 109.22) (end 185.40499 109.22) (width 1) (layer B.Cu) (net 24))
 (segment (start 182.88 106.68) (end 185.40499 106.68) (width 1) (layer B.Cu) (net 25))
 (segment (start 182.88 104.14) (end 185.40499 104.14) (width 1) (layer B.Cu) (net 26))
 (segment (start 182.88 101.6) (end 185.40499 101.6) (width 1) (layer B.Cu) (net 27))
 (segment (start 182.88 99.06) (end 185.40499 99.06) (width 1) (layer B.Cu) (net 28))
 (segment (start 182.88 96.52) (end 185.40499 96.52) (width 1) (layer B.Cu) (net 29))
 (segment (start 170.18 81.28) (end 170.18 86.36) (width 1) (layer B.Cu) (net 2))
 (segment (start 170.18 86.36) (end 172.72 86.36) (width 1) (layer B.Cu) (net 2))
 (segment (start 182.88 93.98) (end 185.40499 93.98) (width 1) (layer B.Cu) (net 30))
 (segment (start 132.08 111.76) (end 132.08 114.3) (width 1) (layer B.Cu) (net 31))
 (segment (start 132.08 114.3) (end 142.24 114.3) (width 1) (layer B.Cu) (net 31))
 (segment (start 142.24 114.3) (end 142.24 116.84) (width 1) (layer B.Cu) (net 31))
 (segment (start 134.62 111.76) (end 134.62 114.3) (width 1) (layer F.Cu) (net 32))
 (segment (start 134.62 114.3) (end 142.24 114.3) (width 1) (layer F.Cu) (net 32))
 (segment (start 142.24 114.3) (end 142.24 111.76) (width 1) (layer F.Cu) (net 32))
 (segment (start 175.26 109.22) (end 172.72 109.22) (width 1) (layer B.Cu) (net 13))
 (segment (start 175.26 106.68) (end 172.72 106.68) (width 1) (layer B.Cu) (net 14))
 (segment (start 175.26 104.14) (end 172.72 104.14) (width 1) (layer B.Cu) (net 15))
 (segment (start 175.26 101.6) (end 172.72 101.6) (width 1) (layer B.Cu) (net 16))
 (segment (start 172.72 99.06) (end 175.26 99.06) (width 1) (layer B.Cu) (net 17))
 (segment (start 172.72 96.52) (end 175.26 96.52) (width 1) (layer B.Cu) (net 18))
 (segment (start 172.72 93.98) (end 175.26 93.98) (width 1) (layer B.Cu) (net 19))
 (segment (start 172.72 91.44) (end 175.26 91.44) (width 1) (layer B.Cu) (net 20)))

